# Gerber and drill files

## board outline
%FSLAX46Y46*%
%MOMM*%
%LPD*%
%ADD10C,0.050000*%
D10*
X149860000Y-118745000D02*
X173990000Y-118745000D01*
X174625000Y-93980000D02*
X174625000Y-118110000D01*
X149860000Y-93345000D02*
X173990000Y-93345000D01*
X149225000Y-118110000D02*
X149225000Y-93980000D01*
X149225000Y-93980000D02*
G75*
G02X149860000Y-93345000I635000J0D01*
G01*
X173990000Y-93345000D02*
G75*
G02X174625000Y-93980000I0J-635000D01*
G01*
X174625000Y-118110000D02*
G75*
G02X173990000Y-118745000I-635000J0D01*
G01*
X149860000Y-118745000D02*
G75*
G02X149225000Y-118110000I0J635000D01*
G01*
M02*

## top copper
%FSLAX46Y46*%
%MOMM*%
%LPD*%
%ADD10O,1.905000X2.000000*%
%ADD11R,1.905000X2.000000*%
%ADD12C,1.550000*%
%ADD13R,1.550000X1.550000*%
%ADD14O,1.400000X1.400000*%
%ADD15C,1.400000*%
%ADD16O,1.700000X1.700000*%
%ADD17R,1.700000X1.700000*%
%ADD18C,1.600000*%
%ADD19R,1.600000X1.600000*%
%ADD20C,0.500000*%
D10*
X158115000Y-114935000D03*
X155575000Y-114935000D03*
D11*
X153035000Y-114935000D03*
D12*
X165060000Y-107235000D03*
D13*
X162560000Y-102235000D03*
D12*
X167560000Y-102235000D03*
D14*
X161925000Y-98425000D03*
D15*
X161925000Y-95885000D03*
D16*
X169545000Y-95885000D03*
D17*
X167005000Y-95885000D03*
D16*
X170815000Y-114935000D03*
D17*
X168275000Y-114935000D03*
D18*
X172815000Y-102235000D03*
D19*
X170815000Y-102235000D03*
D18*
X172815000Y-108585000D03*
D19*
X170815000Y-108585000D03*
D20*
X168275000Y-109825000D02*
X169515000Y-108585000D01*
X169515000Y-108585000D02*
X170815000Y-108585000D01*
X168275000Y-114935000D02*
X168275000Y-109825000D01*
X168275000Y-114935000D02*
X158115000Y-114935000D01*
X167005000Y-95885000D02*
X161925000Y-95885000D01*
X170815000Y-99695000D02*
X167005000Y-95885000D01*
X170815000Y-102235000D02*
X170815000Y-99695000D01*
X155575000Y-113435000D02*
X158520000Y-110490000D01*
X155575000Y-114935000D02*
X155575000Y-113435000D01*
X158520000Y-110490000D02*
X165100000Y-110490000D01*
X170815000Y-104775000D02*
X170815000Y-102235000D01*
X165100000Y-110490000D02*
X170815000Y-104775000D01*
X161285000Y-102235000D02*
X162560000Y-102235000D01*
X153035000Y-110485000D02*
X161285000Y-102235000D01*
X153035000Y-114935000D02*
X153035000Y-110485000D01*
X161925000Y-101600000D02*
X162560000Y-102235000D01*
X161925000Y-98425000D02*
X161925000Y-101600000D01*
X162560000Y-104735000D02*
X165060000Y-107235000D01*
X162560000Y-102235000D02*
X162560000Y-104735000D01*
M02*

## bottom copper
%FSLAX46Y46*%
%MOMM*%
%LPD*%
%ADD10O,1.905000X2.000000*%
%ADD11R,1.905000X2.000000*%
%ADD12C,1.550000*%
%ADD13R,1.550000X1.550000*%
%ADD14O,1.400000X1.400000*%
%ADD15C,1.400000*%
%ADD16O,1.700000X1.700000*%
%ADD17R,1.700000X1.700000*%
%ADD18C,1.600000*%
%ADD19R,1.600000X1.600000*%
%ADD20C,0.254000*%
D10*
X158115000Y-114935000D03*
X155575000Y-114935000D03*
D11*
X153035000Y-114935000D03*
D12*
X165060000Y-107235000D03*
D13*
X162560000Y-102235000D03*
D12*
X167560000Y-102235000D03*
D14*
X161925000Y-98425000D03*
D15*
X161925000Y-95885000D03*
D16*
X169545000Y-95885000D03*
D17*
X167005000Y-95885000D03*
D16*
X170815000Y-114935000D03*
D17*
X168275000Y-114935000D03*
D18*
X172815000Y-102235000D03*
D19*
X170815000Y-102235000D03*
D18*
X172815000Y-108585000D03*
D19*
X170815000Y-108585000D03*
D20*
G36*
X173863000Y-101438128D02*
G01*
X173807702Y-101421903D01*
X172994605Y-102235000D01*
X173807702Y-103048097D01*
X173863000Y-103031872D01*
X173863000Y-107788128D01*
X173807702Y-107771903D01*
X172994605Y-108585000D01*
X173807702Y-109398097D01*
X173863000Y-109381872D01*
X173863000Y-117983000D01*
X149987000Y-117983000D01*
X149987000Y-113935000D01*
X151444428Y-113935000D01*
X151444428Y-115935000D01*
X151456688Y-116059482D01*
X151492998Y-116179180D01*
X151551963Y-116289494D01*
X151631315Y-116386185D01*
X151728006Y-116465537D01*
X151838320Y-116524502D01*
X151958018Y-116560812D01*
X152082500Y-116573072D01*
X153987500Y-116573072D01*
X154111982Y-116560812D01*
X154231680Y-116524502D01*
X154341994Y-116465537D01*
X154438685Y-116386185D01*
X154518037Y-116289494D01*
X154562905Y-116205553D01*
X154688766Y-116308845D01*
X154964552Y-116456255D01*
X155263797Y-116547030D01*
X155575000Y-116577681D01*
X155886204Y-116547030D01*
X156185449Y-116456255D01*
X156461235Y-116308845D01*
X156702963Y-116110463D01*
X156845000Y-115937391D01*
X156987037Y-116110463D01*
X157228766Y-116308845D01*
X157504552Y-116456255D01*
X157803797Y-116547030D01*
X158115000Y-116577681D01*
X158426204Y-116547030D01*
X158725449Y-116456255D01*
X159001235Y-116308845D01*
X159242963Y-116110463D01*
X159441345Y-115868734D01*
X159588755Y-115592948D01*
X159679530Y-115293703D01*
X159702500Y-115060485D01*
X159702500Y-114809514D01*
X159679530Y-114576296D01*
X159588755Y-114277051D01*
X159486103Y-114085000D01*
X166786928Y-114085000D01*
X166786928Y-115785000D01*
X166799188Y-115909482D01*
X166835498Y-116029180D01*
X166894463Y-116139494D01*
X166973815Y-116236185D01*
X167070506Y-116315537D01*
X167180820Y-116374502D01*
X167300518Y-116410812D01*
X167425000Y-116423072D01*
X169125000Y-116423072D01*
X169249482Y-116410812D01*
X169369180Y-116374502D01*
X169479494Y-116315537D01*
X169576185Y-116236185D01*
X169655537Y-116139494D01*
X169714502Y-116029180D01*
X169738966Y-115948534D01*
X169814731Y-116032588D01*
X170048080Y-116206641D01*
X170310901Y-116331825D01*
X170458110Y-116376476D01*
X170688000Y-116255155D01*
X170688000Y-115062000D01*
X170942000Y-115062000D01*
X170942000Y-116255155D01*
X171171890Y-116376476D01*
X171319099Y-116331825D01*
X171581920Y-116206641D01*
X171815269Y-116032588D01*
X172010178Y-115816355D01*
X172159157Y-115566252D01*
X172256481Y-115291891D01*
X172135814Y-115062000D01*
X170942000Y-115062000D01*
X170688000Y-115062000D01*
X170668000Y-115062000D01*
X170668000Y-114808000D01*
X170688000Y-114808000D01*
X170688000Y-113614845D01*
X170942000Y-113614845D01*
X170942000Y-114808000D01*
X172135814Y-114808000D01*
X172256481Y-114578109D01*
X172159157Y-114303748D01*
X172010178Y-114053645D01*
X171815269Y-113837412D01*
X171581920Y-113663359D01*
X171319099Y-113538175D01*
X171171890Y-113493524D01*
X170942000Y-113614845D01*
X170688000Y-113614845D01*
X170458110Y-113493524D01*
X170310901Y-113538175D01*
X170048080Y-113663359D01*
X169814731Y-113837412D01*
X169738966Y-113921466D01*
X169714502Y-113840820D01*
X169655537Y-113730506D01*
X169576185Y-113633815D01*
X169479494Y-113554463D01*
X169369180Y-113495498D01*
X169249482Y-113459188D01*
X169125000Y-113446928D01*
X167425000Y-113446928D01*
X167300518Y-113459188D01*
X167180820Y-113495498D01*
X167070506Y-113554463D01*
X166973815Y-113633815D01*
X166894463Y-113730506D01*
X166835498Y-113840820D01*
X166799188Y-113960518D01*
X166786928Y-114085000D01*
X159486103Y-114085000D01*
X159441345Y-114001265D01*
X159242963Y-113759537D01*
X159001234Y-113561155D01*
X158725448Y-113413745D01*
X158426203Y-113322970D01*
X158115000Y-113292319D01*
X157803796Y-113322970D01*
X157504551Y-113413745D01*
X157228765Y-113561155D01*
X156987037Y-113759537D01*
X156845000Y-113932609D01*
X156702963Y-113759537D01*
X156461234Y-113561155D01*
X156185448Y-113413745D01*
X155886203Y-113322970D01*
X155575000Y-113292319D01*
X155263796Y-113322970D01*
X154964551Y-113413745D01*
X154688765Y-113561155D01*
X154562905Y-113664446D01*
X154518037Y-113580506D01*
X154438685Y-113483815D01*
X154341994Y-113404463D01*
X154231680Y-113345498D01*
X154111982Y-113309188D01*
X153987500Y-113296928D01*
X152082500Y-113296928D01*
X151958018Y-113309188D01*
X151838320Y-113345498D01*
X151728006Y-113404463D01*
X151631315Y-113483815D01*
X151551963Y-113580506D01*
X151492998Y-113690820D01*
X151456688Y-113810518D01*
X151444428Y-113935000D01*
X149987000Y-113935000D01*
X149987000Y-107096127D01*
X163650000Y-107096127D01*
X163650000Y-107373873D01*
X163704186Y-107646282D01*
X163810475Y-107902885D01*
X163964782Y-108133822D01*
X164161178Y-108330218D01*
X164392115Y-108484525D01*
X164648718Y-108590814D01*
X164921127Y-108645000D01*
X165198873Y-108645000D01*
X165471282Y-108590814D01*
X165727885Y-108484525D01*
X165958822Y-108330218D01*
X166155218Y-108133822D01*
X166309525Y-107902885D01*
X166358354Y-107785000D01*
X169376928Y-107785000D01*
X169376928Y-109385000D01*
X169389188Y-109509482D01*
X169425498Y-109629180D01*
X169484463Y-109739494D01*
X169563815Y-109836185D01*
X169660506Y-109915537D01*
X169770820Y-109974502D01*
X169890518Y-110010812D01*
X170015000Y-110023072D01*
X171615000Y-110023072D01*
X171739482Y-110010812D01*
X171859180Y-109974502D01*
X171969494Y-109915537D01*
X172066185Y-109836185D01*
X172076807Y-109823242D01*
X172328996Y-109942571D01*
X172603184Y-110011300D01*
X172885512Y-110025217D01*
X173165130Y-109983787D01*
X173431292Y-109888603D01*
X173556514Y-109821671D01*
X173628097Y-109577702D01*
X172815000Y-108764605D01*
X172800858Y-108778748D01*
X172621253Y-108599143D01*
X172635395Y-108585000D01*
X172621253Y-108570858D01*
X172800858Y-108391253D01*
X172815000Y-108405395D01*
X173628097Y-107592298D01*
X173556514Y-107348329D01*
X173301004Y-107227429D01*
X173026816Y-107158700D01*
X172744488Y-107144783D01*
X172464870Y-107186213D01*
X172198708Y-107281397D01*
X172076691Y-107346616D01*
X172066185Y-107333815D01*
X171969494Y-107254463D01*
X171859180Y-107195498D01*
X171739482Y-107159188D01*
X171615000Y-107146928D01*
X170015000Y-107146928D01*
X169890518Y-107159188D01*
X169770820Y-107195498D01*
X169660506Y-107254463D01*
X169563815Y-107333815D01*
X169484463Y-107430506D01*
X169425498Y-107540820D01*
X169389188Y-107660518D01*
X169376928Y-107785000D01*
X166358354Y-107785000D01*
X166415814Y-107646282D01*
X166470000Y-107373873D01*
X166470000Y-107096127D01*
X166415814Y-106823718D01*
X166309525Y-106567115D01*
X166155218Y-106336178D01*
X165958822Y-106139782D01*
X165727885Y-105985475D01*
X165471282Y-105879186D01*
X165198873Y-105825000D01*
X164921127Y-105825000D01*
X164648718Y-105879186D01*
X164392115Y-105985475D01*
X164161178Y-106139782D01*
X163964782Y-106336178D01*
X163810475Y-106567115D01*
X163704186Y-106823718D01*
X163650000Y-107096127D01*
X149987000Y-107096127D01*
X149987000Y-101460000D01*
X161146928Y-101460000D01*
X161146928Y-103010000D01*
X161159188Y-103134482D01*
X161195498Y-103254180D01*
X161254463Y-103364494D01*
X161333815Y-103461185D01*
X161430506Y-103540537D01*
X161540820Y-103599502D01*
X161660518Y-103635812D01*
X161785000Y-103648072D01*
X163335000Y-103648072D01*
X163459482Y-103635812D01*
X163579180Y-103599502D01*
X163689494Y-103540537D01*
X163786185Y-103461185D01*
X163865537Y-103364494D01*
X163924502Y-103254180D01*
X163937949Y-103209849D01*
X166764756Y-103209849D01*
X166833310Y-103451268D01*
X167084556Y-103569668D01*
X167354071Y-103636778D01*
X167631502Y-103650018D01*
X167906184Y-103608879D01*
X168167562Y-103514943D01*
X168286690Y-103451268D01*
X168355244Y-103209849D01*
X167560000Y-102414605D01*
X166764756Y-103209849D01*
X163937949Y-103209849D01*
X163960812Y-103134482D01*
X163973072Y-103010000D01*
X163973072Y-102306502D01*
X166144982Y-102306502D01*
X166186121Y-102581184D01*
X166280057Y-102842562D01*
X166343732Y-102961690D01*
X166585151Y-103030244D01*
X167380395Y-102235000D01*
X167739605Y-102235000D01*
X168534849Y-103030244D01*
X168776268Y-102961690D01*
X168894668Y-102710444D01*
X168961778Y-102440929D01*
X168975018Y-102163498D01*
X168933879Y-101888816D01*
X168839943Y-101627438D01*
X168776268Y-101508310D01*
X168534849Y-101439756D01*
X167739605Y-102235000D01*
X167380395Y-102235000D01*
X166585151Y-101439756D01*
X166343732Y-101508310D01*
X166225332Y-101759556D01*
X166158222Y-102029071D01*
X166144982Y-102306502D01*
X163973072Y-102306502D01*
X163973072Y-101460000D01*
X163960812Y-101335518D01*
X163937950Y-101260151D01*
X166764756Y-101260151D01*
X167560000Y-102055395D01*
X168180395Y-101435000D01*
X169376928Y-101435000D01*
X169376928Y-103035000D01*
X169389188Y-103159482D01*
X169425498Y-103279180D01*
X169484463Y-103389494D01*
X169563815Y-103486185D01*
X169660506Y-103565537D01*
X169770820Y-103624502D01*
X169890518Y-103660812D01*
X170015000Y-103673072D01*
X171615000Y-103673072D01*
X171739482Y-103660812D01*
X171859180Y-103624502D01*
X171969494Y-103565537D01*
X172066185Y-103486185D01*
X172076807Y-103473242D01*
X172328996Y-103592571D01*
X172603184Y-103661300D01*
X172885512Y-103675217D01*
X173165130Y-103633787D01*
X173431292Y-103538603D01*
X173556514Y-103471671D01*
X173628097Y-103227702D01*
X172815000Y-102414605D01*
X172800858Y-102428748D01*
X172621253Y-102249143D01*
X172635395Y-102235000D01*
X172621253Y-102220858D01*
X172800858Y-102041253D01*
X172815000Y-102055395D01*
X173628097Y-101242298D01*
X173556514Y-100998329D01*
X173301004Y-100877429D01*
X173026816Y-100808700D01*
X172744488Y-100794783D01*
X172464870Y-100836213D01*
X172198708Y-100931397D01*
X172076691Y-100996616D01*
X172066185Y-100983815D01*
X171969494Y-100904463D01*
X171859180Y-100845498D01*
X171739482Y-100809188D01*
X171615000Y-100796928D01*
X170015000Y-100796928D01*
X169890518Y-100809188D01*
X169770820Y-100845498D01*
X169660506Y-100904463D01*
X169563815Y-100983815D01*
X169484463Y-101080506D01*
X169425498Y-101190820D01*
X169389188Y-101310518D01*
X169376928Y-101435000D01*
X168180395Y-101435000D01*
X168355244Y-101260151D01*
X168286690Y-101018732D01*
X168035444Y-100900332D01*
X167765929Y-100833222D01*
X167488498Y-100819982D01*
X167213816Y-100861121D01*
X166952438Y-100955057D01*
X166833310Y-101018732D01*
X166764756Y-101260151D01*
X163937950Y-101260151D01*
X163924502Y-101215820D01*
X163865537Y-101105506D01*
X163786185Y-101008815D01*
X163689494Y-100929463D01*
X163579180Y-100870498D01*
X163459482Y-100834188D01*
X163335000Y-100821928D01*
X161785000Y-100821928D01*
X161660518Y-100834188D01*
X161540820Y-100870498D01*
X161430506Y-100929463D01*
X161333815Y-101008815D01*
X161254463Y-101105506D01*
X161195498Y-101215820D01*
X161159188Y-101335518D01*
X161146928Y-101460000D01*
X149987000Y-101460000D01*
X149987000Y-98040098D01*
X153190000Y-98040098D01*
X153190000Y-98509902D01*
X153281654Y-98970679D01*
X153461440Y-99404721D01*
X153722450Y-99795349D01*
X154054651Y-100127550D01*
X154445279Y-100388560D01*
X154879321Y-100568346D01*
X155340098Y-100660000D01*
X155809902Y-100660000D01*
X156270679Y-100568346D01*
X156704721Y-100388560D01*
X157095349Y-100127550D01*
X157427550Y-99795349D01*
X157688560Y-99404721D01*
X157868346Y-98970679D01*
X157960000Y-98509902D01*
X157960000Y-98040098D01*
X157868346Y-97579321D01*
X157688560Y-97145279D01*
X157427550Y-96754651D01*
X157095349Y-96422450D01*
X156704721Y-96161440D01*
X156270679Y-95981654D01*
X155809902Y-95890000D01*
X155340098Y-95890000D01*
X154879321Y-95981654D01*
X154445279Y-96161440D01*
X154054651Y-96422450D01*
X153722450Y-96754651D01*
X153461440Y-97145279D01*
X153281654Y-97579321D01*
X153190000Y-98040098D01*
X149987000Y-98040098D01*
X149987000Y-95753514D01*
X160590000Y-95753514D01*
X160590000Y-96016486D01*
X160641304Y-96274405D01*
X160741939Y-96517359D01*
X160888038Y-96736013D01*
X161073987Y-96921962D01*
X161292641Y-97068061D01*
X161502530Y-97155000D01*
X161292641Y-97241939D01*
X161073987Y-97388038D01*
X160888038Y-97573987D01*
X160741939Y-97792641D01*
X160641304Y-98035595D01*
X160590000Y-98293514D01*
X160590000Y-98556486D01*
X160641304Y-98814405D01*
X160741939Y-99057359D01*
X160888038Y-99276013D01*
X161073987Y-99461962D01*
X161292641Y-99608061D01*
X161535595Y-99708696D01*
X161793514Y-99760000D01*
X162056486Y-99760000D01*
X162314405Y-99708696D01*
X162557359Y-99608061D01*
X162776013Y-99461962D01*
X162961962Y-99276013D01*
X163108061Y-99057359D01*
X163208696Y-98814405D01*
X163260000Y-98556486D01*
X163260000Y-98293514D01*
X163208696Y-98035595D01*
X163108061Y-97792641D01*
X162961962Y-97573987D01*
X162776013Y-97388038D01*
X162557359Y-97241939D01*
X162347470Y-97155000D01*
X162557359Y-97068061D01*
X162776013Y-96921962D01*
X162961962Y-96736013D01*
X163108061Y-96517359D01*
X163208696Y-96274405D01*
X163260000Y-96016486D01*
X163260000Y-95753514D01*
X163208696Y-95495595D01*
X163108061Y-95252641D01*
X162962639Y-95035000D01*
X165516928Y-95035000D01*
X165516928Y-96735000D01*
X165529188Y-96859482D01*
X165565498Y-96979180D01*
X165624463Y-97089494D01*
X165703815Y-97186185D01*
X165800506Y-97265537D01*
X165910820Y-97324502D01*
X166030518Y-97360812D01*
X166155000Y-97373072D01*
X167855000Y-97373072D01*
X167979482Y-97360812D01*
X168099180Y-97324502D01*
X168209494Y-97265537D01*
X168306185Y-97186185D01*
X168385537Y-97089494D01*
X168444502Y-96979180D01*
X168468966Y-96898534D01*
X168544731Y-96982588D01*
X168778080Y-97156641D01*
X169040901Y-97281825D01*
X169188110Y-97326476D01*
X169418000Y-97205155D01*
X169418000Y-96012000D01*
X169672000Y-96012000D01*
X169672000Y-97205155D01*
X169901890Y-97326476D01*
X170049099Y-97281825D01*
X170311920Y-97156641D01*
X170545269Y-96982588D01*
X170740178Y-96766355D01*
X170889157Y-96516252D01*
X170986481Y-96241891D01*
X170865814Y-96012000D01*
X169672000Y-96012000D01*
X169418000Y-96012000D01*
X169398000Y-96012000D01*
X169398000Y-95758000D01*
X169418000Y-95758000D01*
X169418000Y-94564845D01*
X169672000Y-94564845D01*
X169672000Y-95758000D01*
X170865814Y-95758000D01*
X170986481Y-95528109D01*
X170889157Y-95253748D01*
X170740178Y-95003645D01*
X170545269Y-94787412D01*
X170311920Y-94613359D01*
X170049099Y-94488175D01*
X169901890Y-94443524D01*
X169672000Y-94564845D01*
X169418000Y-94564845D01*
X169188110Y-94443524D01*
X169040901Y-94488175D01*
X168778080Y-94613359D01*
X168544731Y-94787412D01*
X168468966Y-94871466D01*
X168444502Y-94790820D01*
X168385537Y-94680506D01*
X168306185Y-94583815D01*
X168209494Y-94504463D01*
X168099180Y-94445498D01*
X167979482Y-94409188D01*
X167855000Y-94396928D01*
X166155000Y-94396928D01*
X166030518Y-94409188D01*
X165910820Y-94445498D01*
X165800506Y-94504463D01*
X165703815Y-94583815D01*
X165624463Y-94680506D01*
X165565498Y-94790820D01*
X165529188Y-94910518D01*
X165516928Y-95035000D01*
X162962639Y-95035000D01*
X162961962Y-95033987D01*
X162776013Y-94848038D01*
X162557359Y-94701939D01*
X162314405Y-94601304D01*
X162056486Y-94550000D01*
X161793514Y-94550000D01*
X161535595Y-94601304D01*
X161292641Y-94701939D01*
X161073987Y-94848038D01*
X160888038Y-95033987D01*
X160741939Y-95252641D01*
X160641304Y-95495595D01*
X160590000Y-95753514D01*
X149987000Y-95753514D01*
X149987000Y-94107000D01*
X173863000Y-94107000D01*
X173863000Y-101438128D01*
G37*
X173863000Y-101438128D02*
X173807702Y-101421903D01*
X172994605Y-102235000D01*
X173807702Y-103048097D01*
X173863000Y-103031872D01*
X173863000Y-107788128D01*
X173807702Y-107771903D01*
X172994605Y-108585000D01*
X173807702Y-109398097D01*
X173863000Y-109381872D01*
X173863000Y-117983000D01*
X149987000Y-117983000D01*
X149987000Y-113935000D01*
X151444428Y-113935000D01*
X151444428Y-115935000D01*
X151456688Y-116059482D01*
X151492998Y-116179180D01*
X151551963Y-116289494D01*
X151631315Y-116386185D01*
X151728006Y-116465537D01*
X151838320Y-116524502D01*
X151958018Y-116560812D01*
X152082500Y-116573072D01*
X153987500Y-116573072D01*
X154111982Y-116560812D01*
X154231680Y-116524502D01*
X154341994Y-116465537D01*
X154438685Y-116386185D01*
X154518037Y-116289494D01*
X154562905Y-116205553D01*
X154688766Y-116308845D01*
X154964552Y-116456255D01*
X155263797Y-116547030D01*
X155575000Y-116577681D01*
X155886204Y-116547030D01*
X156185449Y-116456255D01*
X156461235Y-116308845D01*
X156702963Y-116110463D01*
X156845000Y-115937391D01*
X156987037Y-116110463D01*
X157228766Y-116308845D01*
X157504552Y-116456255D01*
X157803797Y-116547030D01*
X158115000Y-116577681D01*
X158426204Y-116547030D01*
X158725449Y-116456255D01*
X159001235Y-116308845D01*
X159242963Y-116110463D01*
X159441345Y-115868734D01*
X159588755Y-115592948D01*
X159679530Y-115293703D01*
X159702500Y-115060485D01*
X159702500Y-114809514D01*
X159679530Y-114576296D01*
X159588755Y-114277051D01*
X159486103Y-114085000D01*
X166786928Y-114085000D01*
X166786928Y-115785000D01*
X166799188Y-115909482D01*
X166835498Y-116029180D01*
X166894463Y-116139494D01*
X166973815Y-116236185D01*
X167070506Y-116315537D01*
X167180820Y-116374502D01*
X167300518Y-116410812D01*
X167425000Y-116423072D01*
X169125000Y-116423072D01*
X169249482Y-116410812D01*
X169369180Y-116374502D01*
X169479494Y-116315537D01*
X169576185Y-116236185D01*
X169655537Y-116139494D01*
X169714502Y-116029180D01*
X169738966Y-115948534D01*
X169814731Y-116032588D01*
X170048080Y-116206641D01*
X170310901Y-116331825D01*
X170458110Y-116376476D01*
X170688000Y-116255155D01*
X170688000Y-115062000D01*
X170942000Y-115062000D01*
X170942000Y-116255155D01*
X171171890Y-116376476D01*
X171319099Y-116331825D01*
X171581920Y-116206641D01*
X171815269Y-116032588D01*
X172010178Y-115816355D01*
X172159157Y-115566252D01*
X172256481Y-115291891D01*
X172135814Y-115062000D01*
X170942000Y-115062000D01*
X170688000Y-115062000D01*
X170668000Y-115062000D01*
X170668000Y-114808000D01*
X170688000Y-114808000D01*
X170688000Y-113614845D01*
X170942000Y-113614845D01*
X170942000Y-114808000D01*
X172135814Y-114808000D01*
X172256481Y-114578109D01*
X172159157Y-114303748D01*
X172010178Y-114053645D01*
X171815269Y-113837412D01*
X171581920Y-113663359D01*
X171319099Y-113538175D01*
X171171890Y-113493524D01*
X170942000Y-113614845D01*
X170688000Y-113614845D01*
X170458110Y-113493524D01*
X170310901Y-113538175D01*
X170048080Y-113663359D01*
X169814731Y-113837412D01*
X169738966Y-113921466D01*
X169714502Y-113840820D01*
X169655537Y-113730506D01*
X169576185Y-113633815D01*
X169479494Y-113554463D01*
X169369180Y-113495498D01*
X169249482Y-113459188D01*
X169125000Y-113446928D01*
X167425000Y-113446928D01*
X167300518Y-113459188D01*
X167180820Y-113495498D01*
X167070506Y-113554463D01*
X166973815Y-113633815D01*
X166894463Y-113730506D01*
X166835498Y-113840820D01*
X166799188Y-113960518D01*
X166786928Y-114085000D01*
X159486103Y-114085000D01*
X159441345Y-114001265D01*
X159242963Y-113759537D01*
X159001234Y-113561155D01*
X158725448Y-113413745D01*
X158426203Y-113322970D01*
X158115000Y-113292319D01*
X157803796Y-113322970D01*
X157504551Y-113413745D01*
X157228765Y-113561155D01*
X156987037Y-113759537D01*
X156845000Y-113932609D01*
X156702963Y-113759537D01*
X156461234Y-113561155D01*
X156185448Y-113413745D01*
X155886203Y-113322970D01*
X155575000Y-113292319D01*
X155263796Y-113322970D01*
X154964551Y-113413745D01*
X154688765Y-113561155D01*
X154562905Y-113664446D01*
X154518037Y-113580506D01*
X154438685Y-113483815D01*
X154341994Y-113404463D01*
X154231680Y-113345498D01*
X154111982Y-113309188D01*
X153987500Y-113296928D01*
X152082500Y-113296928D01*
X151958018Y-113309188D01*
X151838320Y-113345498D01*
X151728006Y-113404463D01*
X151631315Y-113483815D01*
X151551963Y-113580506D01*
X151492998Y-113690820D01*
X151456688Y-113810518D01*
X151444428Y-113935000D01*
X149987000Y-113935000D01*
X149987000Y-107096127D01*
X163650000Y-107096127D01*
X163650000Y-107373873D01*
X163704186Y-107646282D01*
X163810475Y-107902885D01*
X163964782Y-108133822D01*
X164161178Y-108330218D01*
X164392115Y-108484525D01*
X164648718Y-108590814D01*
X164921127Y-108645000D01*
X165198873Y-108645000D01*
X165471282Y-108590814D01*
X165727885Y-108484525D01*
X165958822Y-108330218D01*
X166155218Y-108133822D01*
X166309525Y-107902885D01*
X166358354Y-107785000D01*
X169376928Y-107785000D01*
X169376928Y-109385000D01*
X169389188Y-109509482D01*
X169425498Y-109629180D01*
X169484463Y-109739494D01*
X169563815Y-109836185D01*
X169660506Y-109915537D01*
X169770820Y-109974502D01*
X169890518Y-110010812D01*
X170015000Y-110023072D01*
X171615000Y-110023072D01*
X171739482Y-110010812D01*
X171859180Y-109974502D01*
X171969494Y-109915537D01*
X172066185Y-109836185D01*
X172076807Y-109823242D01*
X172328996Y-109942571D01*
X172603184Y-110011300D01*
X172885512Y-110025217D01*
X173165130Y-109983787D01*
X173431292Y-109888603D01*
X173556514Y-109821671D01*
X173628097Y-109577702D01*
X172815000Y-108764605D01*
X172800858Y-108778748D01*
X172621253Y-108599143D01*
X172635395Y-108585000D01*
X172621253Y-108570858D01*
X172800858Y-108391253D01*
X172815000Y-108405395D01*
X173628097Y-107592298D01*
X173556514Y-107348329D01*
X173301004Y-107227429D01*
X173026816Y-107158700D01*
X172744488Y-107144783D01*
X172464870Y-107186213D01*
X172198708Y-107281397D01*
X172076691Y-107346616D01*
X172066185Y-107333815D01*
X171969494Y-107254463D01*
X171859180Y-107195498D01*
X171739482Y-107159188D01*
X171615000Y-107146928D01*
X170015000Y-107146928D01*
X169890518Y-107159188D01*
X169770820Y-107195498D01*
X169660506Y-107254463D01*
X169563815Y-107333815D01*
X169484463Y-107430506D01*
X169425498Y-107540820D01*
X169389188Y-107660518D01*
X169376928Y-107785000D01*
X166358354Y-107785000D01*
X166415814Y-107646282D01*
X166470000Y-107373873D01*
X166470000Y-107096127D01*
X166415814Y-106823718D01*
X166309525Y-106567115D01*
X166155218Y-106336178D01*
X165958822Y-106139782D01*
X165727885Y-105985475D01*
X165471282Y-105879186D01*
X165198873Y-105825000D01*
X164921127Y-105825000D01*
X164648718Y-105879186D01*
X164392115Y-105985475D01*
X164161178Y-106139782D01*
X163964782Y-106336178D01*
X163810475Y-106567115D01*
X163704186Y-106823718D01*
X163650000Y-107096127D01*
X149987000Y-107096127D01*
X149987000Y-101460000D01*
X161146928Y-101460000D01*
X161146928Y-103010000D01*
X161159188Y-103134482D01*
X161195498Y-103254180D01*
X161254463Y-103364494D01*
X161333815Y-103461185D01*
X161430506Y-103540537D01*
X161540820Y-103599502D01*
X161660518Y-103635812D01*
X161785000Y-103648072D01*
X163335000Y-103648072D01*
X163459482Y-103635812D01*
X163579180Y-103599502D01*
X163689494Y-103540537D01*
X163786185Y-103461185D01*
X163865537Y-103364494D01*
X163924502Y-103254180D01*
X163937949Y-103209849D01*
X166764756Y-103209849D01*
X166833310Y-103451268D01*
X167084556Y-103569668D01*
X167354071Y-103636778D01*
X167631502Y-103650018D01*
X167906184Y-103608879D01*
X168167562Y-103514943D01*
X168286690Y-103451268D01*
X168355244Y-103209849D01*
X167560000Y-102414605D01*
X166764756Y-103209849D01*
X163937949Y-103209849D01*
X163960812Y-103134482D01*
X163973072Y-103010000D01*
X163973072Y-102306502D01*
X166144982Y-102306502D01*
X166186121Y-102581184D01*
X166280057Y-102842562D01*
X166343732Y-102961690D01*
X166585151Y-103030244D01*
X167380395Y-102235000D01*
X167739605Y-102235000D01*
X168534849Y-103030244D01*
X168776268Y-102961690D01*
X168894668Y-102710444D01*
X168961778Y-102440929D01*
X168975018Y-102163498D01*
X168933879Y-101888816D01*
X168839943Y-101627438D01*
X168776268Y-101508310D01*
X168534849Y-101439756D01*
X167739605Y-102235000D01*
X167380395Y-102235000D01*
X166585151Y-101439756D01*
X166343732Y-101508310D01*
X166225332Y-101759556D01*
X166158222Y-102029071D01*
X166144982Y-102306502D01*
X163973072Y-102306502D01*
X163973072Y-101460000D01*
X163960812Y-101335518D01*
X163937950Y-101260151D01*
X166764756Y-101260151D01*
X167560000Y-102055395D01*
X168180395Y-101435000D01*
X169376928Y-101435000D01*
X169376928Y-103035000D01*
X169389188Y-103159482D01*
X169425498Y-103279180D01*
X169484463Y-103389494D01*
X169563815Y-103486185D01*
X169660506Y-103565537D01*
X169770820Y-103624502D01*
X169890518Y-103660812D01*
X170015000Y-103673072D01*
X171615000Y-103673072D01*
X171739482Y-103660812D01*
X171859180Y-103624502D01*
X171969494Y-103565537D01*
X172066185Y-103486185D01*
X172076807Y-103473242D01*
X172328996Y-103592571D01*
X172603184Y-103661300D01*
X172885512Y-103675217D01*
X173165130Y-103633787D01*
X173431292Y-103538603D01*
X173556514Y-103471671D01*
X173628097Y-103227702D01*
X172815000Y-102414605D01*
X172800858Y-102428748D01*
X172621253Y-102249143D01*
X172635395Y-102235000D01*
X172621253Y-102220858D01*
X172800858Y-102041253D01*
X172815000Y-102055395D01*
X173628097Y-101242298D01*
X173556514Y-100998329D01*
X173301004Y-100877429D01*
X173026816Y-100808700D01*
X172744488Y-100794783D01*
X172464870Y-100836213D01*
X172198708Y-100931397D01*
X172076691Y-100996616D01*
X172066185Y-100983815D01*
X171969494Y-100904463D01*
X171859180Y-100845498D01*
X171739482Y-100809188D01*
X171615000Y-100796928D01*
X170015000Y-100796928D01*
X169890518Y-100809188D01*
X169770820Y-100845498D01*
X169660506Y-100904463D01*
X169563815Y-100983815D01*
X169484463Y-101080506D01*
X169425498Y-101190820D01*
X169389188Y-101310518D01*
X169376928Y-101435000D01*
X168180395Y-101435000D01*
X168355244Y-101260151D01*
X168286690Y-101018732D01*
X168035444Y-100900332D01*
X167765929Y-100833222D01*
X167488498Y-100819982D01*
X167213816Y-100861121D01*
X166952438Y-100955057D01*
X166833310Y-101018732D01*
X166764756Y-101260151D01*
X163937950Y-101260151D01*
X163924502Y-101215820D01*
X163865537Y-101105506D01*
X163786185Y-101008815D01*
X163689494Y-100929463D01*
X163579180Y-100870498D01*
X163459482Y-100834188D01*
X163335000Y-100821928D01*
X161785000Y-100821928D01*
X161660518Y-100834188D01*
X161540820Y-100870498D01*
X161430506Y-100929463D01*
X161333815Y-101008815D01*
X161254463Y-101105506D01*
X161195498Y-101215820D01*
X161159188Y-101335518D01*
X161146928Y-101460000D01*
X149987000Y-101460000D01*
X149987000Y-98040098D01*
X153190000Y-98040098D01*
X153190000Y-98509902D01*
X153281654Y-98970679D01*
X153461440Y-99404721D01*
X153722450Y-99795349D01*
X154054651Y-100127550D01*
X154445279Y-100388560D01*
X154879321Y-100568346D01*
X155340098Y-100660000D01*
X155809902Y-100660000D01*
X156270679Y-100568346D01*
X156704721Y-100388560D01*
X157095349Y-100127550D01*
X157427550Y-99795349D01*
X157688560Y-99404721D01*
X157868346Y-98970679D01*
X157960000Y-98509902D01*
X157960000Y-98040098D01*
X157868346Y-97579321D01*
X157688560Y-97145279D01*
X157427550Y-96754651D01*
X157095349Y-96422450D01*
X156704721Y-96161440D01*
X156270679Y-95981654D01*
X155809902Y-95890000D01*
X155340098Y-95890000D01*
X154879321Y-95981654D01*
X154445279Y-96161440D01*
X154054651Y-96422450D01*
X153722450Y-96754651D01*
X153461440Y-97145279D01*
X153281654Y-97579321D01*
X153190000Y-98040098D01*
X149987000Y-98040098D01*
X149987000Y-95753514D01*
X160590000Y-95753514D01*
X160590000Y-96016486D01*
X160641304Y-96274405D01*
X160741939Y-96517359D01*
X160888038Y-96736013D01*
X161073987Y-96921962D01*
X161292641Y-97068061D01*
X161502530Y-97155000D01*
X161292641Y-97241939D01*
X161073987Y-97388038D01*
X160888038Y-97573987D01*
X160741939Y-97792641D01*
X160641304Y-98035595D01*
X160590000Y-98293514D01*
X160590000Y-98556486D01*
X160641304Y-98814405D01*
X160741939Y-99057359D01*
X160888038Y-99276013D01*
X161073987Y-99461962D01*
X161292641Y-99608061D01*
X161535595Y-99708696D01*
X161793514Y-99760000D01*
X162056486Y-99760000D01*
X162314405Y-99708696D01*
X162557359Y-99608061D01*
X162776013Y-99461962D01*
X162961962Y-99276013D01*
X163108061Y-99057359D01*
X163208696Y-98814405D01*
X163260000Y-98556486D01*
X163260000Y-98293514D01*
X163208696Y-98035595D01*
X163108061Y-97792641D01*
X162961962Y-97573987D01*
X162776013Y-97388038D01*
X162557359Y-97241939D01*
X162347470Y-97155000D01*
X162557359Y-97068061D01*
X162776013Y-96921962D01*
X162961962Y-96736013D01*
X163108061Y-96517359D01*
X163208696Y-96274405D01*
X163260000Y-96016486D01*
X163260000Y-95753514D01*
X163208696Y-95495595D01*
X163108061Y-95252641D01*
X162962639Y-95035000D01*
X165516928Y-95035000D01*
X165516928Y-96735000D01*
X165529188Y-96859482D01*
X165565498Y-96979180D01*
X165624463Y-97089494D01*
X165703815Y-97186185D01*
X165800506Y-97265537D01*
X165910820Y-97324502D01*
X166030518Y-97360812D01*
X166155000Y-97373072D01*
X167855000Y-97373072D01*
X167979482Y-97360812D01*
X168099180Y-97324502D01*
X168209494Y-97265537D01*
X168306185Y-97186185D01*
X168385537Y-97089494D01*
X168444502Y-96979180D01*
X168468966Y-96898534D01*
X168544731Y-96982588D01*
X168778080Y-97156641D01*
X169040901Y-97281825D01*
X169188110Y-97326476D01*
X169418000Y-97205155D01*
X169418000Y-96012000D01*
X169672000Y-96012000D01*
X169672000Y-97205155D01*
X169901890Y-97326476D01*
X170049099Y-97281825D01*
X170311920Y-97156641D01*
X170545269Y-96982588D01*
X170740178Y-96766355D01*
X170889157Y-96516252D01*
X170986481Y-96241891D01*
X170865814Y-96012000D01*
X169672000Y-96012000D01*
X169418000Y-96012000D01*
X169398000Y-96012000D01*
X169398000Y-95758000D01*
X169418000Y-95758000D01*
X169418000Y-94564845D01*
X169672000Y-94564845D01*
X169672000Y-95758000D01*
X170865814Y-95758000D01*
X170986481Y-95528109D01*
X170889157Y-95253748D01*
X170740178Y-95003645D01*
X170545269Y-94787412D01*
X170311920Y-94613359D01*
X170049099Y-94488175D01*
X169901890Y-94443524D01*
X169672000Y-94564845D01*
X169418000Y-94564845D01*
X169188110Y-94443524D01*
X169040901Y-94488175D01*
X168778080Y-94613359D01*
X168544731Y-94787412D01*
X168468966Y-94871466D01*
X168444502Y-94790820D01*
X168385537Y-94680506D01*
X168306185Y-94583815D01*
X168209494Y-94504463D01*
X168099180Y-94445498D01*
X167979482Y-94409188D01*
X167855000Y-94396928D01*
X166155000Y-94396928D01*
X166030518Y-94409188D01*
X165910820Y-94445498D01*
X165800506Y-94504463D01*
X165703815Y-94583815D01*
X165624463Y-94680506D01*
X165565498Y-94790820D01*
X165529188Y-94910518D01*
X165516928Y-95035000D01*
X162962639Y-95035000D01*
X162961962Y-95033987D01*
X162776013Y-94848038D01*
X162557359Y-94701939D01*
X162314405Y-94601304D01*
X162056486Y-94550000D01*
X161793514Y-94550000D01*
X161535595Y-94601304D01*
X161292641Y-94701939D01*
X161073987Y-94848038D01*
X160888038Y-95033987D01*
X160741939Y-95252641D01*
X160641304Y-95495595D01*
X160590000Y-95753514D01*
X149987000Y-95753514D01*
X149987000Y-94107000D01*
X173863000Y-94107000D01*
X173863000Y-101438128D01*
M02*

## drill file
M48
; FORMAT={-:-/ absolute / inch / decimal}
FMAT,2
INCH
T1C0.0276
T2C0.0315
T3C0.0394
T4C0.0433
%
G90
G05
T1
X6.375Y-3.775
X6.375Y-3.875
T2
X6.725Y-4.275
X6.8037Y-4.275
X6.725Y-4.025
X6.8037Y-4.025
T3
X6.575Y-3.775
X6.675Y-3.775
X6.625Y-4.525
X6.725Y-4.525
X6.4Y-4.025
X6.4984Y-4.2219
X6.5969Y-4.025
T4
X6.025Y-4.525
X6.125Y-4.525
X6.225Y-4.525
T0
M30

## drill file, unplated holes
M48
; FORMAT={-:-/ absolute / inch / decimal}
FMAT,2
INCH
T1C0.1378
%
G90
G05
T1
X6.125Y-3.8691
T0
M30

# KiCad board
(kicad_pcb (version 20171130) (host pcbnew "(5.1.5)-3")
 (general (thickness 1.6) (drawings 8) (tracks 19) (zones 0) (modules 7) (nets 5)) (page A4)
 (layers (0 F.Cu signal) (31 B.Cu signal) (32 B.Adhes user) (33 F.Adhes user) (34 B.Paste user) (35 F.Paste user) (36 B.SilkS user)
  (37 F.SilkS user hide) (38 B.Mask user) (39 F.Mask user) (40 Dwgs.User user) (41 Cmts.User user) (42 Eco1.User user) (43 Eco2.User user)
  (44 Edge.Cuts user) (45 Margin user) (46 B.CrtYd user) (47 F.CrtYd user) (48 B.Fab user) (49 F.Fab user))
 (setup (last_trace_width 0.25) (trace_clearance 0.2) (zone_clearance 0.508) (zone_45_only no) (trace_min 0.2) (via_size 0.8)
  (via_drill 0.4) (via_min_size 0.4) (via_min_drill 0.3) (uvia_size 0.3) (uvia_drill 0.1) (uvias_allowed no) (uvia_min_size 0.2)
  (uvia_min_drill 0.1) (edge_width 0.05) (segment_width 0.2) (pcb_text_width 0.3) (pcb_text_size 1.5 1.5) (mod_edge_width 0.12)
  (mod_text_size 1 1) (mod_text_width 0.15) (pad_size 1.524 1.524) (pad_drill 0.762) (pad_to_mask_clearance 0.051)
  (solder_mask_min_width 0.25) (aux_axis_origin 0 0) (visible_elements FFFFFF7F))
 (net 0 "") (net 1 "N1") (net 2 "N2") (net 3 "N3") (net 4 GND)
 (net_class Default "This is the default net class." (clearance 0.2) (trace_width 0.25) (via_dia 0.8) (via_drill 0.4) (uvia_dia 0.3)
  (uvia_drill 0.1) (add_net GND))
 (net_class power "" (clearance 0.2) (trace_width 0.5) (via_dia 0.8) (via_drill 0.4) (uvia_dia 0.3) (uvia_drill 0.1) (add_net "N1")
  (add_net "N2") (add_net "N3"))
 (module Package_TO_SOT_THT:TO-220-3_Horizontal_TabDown (layer F.Cu) (at 153.035 114.935)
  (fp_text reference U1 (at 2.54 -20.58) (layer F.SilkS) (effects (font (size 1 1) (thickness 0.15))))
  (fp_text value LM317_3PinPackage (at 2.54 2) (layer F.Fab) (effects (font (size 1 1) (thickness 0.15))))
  (pad 3 thru_hole oval (at 5.08 0) (size 1.905 2) (drill 1.1) (layers *.Cu *.Mask) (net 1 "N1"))
  (pad 2 thru_hole oval (at 2.54 0) (size 1.905 2) (drill 1.1) (layers *.Cu *.Mask) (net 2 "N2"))
  (pad 1 thru_hole rect (at 0 0) (size 1.905 2) (drill 1.1) (layers *.Cu *.Mask) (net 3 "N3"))
  (pad "" np_thru_hole oval (at 2.54 -16.66) (size 3.5 3.5) (drill 3.5) (layers *.Cu *.Mask)))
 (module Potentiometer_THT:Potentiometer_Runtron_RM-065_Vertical (layer F.Cu) (at 162.56 102.235)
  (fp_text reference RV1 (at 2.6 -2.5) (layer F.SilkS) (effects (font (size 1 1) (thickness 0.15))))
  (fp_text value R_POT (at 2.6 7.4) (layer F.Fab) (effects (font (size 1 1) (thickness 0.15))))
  (pad 2 thru_hole circle (at 2.5 5) (size 1.55 1.55) (drill 1) (layers *.Cu *.Mask) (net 3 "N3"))
  (pad 1 thru_hole rect (at 0 0) (size 1.55 1.55) (drill 1) (layers *.Cu *.Mask) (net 3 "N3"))
  (pad 3 thru_hole circle (at 5 0) (size 1.55 1.55) (drill 1) (layers *.Cu *.Mask) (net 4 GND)))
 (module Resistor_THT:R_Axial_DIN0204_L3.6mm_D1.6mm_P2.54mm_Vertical (layer F.Cu) (at 161.925 95.885 270)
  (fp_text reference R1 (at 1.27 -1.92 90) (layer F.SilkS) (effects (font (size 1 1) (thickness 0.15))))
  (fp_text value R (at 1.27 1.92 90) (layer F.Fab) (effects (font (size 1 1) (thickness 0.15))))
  (pad 2 thru_hole oval (at 2.54 0 270) (size 1.4 1.4) (drill 0.7) (layers *.Cu *.Mask) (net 3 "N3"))
  (pad 1 thru_hole circle (at 0 0 270) (size 1.4 1.4) (drill 0.7) (layers *.Cu *.Mask) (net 2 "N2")))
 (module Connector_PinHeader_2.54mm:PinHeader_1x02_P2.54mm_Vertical (layer F.Cu) (at 167.005 95.885 90)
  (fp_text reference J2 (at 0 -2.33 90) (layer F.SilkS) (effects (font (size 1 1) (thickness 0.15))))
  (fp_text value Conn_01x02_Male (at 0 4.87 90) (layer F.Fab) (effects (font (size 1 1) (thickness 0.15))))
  (pad 2 thru_hole oval (at 0 2.54 90) (size 1.7 1.7) (drill 1) (layers *.Cu *.Mask) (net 4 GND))
  (pad 1 thru_hole rect (at 0 0 90) (size 1.7 1.7) (drill 1) (layers *.Cu *.Mask) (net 2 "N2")))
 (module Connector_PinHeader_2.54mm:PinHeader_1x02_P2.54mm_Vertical (layer F.Cu) (at 168.275 114.935 90)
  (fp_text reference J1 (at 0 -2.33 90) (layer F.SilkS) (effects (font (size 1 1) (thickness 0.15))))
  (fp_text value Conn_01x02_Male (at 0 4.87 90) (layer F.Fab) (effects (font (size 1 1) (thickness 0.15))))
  (pad 2 thru_hole oval (at 0 2.54 90) (size 1.7 1.7) (drill 1) (layers *.Cu *.Mask) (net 4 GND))
  (pad 1 thru_hole rect (at 0 0 90) (size 1.7 1.7) (drill 1) (layers *.Cu *.Mask) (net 1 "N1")))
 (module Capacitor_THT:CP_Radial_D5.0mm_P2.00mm (layer F.Cu) (at 170.815 102.235)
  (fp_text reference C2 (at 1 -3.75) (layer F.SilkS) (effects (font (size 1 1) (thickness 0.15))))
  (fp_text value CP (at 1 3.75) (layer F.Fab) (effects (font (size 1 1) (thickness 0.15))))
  (pad 2 thru_hole circle (at 2 0) (size 1.6 1.6) (drill 0.8) (layers *.Cu *.Mask) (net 4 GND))
  (pad 1 thru_hole rect (at 0 0) (size 1.6 1.6) (drill 0.8) (layers *.Cu *.Mask) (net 2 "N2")))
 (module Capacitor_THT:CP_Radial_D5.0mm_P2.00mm (layer F.Cu) (at 170.815 108.585)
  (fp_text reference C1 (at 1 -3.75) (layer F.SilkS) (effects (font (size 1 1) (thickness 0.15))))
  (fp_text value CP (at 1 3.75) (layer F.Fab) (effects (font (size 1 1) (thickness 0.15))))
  (pad 2 thru_hole circle (at 2 0) (size 1.6 1.6) (drill 0.8) (layers *.Cu *.Mask) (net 4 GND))
  (pad 1 thru_hole rect (at 0 0) (size 1.6 1.6) (drill 0.8) (layers *.Cu *.Mask) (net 1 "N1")))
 (gr_line (start 149.86 118.745) (end 173.99 118.745) (layer Edge.Cuts) (width 0.05))
 (gr_line (start 174.625 93.98) (end 174.625 118.11) (layer Edge.Cuts) (width 0.05))
 (gr_line (start 149.86 93.345) (end 173.99 93.345) (layer Edge.Cuts) (width 0.05))
 (gr_line (start 149.225 118.11) (end 149.225 93.98) (layer Edge.Cuts) (width 0.05))
 (gr_arc (start 149.86 93.98) (end 149.86 93.345) (angle -90) (layer Edge.Cuts) (width 0.05))
 (gr_arc (start 173.99 93.98) (end 174.625 93.98) (angle -90) (layer Edge.Cuts) (width 0.05))
 (gr_arc (start 173.99 118.11) (end 173.99 118.745) (angle -90) (layer Edge.Cuts) (width 0.05))
 (gr_arc (start 149.86 118.11) (end 149.225 118.11) (angle -90) (layer Edge.Cuts) (width 0.05))
 (segment (start 168.275 109.825) (end 169.515 108.585) (width 0.5) (layer F.Cu) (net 1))
 (segment (start 169.515 108.585) (end 170.815 108.585) (width 0.5) (layer F.Cu) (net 1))
 (segment (start 168.275 114.935) (end 168.275 109.825) (width 0.5) (layer F.Cu) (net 1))
 (segment (start 168.275 114.935) (end 158.115 114.935) (width 0.5) (layer F.Cu) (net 1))
 (segment (start 167.005 95.885) (end 161.925 95.885) (width 0.5) (layer F.Cu) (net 2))
 (segment (start 170.815 99.695) (end 167.005 95.885) (width 0.5) (layer F.Cu) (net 2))
 (segment (start 170.815 102.235) (end 170.815 99.695) (width 0.5) (layer F.Cu) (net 2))
 (segment (start 155.575 113.435) (end 158.52 110.49) (width 0.5) (layer F.Cu) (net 2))
 (segment (start 155.575 114.935) (end 155.575 113.435) (width 0.5) (layer F.Cu) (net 2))
 (segment (start 158.52 110.49) (end 165.1 110.49) (width 0.5) (layer F.Cu) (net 2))
 (segment (start 170.815 104.775) (end 170.815 102.235) (width 0.5) (layer F.Cu) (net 2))
 (segment (start 165.1 110.49) (end 170.815 104.775) (width 0.5) (layer F.Cu) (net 2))
 (segment (start 161.285 102.235) (end 162.56 102.235) (width 0.5) (layer F.Cu) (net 3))
 (segment (start 153.035 110.485) (end 161.285 102.235) (width 0.5) (layer F.Cu) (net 3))
 (segment (start 153.035 114.935) (end 153.035 110.485) (width 0.5) (layer F.Cu) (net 3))
 (segment (start 161.925 101.6) (end 162.56 102.235) (width 0.5) (layer F.Cu) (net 3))
 (segment (start 161.925 98.425) (end 161.925 101.6) (width 0.5) (layer F.Cu) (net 3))
 (segment (start 162.56 104.735) (end 165.06 107.235) (width 0.5) (layer F.Cu) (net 3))
 (segment (start 162.56 102.235) (end 162.56 104.735) (width 0.5) (layer F.Cu) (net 3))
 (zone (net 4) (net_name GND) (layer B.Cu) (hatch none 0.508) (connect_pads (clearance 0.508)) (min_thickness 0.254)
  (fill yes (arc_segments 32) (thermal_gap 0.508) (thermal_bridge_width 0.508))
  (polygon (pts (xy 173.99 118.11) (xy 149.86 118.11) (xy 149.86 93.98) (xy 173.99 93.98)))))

